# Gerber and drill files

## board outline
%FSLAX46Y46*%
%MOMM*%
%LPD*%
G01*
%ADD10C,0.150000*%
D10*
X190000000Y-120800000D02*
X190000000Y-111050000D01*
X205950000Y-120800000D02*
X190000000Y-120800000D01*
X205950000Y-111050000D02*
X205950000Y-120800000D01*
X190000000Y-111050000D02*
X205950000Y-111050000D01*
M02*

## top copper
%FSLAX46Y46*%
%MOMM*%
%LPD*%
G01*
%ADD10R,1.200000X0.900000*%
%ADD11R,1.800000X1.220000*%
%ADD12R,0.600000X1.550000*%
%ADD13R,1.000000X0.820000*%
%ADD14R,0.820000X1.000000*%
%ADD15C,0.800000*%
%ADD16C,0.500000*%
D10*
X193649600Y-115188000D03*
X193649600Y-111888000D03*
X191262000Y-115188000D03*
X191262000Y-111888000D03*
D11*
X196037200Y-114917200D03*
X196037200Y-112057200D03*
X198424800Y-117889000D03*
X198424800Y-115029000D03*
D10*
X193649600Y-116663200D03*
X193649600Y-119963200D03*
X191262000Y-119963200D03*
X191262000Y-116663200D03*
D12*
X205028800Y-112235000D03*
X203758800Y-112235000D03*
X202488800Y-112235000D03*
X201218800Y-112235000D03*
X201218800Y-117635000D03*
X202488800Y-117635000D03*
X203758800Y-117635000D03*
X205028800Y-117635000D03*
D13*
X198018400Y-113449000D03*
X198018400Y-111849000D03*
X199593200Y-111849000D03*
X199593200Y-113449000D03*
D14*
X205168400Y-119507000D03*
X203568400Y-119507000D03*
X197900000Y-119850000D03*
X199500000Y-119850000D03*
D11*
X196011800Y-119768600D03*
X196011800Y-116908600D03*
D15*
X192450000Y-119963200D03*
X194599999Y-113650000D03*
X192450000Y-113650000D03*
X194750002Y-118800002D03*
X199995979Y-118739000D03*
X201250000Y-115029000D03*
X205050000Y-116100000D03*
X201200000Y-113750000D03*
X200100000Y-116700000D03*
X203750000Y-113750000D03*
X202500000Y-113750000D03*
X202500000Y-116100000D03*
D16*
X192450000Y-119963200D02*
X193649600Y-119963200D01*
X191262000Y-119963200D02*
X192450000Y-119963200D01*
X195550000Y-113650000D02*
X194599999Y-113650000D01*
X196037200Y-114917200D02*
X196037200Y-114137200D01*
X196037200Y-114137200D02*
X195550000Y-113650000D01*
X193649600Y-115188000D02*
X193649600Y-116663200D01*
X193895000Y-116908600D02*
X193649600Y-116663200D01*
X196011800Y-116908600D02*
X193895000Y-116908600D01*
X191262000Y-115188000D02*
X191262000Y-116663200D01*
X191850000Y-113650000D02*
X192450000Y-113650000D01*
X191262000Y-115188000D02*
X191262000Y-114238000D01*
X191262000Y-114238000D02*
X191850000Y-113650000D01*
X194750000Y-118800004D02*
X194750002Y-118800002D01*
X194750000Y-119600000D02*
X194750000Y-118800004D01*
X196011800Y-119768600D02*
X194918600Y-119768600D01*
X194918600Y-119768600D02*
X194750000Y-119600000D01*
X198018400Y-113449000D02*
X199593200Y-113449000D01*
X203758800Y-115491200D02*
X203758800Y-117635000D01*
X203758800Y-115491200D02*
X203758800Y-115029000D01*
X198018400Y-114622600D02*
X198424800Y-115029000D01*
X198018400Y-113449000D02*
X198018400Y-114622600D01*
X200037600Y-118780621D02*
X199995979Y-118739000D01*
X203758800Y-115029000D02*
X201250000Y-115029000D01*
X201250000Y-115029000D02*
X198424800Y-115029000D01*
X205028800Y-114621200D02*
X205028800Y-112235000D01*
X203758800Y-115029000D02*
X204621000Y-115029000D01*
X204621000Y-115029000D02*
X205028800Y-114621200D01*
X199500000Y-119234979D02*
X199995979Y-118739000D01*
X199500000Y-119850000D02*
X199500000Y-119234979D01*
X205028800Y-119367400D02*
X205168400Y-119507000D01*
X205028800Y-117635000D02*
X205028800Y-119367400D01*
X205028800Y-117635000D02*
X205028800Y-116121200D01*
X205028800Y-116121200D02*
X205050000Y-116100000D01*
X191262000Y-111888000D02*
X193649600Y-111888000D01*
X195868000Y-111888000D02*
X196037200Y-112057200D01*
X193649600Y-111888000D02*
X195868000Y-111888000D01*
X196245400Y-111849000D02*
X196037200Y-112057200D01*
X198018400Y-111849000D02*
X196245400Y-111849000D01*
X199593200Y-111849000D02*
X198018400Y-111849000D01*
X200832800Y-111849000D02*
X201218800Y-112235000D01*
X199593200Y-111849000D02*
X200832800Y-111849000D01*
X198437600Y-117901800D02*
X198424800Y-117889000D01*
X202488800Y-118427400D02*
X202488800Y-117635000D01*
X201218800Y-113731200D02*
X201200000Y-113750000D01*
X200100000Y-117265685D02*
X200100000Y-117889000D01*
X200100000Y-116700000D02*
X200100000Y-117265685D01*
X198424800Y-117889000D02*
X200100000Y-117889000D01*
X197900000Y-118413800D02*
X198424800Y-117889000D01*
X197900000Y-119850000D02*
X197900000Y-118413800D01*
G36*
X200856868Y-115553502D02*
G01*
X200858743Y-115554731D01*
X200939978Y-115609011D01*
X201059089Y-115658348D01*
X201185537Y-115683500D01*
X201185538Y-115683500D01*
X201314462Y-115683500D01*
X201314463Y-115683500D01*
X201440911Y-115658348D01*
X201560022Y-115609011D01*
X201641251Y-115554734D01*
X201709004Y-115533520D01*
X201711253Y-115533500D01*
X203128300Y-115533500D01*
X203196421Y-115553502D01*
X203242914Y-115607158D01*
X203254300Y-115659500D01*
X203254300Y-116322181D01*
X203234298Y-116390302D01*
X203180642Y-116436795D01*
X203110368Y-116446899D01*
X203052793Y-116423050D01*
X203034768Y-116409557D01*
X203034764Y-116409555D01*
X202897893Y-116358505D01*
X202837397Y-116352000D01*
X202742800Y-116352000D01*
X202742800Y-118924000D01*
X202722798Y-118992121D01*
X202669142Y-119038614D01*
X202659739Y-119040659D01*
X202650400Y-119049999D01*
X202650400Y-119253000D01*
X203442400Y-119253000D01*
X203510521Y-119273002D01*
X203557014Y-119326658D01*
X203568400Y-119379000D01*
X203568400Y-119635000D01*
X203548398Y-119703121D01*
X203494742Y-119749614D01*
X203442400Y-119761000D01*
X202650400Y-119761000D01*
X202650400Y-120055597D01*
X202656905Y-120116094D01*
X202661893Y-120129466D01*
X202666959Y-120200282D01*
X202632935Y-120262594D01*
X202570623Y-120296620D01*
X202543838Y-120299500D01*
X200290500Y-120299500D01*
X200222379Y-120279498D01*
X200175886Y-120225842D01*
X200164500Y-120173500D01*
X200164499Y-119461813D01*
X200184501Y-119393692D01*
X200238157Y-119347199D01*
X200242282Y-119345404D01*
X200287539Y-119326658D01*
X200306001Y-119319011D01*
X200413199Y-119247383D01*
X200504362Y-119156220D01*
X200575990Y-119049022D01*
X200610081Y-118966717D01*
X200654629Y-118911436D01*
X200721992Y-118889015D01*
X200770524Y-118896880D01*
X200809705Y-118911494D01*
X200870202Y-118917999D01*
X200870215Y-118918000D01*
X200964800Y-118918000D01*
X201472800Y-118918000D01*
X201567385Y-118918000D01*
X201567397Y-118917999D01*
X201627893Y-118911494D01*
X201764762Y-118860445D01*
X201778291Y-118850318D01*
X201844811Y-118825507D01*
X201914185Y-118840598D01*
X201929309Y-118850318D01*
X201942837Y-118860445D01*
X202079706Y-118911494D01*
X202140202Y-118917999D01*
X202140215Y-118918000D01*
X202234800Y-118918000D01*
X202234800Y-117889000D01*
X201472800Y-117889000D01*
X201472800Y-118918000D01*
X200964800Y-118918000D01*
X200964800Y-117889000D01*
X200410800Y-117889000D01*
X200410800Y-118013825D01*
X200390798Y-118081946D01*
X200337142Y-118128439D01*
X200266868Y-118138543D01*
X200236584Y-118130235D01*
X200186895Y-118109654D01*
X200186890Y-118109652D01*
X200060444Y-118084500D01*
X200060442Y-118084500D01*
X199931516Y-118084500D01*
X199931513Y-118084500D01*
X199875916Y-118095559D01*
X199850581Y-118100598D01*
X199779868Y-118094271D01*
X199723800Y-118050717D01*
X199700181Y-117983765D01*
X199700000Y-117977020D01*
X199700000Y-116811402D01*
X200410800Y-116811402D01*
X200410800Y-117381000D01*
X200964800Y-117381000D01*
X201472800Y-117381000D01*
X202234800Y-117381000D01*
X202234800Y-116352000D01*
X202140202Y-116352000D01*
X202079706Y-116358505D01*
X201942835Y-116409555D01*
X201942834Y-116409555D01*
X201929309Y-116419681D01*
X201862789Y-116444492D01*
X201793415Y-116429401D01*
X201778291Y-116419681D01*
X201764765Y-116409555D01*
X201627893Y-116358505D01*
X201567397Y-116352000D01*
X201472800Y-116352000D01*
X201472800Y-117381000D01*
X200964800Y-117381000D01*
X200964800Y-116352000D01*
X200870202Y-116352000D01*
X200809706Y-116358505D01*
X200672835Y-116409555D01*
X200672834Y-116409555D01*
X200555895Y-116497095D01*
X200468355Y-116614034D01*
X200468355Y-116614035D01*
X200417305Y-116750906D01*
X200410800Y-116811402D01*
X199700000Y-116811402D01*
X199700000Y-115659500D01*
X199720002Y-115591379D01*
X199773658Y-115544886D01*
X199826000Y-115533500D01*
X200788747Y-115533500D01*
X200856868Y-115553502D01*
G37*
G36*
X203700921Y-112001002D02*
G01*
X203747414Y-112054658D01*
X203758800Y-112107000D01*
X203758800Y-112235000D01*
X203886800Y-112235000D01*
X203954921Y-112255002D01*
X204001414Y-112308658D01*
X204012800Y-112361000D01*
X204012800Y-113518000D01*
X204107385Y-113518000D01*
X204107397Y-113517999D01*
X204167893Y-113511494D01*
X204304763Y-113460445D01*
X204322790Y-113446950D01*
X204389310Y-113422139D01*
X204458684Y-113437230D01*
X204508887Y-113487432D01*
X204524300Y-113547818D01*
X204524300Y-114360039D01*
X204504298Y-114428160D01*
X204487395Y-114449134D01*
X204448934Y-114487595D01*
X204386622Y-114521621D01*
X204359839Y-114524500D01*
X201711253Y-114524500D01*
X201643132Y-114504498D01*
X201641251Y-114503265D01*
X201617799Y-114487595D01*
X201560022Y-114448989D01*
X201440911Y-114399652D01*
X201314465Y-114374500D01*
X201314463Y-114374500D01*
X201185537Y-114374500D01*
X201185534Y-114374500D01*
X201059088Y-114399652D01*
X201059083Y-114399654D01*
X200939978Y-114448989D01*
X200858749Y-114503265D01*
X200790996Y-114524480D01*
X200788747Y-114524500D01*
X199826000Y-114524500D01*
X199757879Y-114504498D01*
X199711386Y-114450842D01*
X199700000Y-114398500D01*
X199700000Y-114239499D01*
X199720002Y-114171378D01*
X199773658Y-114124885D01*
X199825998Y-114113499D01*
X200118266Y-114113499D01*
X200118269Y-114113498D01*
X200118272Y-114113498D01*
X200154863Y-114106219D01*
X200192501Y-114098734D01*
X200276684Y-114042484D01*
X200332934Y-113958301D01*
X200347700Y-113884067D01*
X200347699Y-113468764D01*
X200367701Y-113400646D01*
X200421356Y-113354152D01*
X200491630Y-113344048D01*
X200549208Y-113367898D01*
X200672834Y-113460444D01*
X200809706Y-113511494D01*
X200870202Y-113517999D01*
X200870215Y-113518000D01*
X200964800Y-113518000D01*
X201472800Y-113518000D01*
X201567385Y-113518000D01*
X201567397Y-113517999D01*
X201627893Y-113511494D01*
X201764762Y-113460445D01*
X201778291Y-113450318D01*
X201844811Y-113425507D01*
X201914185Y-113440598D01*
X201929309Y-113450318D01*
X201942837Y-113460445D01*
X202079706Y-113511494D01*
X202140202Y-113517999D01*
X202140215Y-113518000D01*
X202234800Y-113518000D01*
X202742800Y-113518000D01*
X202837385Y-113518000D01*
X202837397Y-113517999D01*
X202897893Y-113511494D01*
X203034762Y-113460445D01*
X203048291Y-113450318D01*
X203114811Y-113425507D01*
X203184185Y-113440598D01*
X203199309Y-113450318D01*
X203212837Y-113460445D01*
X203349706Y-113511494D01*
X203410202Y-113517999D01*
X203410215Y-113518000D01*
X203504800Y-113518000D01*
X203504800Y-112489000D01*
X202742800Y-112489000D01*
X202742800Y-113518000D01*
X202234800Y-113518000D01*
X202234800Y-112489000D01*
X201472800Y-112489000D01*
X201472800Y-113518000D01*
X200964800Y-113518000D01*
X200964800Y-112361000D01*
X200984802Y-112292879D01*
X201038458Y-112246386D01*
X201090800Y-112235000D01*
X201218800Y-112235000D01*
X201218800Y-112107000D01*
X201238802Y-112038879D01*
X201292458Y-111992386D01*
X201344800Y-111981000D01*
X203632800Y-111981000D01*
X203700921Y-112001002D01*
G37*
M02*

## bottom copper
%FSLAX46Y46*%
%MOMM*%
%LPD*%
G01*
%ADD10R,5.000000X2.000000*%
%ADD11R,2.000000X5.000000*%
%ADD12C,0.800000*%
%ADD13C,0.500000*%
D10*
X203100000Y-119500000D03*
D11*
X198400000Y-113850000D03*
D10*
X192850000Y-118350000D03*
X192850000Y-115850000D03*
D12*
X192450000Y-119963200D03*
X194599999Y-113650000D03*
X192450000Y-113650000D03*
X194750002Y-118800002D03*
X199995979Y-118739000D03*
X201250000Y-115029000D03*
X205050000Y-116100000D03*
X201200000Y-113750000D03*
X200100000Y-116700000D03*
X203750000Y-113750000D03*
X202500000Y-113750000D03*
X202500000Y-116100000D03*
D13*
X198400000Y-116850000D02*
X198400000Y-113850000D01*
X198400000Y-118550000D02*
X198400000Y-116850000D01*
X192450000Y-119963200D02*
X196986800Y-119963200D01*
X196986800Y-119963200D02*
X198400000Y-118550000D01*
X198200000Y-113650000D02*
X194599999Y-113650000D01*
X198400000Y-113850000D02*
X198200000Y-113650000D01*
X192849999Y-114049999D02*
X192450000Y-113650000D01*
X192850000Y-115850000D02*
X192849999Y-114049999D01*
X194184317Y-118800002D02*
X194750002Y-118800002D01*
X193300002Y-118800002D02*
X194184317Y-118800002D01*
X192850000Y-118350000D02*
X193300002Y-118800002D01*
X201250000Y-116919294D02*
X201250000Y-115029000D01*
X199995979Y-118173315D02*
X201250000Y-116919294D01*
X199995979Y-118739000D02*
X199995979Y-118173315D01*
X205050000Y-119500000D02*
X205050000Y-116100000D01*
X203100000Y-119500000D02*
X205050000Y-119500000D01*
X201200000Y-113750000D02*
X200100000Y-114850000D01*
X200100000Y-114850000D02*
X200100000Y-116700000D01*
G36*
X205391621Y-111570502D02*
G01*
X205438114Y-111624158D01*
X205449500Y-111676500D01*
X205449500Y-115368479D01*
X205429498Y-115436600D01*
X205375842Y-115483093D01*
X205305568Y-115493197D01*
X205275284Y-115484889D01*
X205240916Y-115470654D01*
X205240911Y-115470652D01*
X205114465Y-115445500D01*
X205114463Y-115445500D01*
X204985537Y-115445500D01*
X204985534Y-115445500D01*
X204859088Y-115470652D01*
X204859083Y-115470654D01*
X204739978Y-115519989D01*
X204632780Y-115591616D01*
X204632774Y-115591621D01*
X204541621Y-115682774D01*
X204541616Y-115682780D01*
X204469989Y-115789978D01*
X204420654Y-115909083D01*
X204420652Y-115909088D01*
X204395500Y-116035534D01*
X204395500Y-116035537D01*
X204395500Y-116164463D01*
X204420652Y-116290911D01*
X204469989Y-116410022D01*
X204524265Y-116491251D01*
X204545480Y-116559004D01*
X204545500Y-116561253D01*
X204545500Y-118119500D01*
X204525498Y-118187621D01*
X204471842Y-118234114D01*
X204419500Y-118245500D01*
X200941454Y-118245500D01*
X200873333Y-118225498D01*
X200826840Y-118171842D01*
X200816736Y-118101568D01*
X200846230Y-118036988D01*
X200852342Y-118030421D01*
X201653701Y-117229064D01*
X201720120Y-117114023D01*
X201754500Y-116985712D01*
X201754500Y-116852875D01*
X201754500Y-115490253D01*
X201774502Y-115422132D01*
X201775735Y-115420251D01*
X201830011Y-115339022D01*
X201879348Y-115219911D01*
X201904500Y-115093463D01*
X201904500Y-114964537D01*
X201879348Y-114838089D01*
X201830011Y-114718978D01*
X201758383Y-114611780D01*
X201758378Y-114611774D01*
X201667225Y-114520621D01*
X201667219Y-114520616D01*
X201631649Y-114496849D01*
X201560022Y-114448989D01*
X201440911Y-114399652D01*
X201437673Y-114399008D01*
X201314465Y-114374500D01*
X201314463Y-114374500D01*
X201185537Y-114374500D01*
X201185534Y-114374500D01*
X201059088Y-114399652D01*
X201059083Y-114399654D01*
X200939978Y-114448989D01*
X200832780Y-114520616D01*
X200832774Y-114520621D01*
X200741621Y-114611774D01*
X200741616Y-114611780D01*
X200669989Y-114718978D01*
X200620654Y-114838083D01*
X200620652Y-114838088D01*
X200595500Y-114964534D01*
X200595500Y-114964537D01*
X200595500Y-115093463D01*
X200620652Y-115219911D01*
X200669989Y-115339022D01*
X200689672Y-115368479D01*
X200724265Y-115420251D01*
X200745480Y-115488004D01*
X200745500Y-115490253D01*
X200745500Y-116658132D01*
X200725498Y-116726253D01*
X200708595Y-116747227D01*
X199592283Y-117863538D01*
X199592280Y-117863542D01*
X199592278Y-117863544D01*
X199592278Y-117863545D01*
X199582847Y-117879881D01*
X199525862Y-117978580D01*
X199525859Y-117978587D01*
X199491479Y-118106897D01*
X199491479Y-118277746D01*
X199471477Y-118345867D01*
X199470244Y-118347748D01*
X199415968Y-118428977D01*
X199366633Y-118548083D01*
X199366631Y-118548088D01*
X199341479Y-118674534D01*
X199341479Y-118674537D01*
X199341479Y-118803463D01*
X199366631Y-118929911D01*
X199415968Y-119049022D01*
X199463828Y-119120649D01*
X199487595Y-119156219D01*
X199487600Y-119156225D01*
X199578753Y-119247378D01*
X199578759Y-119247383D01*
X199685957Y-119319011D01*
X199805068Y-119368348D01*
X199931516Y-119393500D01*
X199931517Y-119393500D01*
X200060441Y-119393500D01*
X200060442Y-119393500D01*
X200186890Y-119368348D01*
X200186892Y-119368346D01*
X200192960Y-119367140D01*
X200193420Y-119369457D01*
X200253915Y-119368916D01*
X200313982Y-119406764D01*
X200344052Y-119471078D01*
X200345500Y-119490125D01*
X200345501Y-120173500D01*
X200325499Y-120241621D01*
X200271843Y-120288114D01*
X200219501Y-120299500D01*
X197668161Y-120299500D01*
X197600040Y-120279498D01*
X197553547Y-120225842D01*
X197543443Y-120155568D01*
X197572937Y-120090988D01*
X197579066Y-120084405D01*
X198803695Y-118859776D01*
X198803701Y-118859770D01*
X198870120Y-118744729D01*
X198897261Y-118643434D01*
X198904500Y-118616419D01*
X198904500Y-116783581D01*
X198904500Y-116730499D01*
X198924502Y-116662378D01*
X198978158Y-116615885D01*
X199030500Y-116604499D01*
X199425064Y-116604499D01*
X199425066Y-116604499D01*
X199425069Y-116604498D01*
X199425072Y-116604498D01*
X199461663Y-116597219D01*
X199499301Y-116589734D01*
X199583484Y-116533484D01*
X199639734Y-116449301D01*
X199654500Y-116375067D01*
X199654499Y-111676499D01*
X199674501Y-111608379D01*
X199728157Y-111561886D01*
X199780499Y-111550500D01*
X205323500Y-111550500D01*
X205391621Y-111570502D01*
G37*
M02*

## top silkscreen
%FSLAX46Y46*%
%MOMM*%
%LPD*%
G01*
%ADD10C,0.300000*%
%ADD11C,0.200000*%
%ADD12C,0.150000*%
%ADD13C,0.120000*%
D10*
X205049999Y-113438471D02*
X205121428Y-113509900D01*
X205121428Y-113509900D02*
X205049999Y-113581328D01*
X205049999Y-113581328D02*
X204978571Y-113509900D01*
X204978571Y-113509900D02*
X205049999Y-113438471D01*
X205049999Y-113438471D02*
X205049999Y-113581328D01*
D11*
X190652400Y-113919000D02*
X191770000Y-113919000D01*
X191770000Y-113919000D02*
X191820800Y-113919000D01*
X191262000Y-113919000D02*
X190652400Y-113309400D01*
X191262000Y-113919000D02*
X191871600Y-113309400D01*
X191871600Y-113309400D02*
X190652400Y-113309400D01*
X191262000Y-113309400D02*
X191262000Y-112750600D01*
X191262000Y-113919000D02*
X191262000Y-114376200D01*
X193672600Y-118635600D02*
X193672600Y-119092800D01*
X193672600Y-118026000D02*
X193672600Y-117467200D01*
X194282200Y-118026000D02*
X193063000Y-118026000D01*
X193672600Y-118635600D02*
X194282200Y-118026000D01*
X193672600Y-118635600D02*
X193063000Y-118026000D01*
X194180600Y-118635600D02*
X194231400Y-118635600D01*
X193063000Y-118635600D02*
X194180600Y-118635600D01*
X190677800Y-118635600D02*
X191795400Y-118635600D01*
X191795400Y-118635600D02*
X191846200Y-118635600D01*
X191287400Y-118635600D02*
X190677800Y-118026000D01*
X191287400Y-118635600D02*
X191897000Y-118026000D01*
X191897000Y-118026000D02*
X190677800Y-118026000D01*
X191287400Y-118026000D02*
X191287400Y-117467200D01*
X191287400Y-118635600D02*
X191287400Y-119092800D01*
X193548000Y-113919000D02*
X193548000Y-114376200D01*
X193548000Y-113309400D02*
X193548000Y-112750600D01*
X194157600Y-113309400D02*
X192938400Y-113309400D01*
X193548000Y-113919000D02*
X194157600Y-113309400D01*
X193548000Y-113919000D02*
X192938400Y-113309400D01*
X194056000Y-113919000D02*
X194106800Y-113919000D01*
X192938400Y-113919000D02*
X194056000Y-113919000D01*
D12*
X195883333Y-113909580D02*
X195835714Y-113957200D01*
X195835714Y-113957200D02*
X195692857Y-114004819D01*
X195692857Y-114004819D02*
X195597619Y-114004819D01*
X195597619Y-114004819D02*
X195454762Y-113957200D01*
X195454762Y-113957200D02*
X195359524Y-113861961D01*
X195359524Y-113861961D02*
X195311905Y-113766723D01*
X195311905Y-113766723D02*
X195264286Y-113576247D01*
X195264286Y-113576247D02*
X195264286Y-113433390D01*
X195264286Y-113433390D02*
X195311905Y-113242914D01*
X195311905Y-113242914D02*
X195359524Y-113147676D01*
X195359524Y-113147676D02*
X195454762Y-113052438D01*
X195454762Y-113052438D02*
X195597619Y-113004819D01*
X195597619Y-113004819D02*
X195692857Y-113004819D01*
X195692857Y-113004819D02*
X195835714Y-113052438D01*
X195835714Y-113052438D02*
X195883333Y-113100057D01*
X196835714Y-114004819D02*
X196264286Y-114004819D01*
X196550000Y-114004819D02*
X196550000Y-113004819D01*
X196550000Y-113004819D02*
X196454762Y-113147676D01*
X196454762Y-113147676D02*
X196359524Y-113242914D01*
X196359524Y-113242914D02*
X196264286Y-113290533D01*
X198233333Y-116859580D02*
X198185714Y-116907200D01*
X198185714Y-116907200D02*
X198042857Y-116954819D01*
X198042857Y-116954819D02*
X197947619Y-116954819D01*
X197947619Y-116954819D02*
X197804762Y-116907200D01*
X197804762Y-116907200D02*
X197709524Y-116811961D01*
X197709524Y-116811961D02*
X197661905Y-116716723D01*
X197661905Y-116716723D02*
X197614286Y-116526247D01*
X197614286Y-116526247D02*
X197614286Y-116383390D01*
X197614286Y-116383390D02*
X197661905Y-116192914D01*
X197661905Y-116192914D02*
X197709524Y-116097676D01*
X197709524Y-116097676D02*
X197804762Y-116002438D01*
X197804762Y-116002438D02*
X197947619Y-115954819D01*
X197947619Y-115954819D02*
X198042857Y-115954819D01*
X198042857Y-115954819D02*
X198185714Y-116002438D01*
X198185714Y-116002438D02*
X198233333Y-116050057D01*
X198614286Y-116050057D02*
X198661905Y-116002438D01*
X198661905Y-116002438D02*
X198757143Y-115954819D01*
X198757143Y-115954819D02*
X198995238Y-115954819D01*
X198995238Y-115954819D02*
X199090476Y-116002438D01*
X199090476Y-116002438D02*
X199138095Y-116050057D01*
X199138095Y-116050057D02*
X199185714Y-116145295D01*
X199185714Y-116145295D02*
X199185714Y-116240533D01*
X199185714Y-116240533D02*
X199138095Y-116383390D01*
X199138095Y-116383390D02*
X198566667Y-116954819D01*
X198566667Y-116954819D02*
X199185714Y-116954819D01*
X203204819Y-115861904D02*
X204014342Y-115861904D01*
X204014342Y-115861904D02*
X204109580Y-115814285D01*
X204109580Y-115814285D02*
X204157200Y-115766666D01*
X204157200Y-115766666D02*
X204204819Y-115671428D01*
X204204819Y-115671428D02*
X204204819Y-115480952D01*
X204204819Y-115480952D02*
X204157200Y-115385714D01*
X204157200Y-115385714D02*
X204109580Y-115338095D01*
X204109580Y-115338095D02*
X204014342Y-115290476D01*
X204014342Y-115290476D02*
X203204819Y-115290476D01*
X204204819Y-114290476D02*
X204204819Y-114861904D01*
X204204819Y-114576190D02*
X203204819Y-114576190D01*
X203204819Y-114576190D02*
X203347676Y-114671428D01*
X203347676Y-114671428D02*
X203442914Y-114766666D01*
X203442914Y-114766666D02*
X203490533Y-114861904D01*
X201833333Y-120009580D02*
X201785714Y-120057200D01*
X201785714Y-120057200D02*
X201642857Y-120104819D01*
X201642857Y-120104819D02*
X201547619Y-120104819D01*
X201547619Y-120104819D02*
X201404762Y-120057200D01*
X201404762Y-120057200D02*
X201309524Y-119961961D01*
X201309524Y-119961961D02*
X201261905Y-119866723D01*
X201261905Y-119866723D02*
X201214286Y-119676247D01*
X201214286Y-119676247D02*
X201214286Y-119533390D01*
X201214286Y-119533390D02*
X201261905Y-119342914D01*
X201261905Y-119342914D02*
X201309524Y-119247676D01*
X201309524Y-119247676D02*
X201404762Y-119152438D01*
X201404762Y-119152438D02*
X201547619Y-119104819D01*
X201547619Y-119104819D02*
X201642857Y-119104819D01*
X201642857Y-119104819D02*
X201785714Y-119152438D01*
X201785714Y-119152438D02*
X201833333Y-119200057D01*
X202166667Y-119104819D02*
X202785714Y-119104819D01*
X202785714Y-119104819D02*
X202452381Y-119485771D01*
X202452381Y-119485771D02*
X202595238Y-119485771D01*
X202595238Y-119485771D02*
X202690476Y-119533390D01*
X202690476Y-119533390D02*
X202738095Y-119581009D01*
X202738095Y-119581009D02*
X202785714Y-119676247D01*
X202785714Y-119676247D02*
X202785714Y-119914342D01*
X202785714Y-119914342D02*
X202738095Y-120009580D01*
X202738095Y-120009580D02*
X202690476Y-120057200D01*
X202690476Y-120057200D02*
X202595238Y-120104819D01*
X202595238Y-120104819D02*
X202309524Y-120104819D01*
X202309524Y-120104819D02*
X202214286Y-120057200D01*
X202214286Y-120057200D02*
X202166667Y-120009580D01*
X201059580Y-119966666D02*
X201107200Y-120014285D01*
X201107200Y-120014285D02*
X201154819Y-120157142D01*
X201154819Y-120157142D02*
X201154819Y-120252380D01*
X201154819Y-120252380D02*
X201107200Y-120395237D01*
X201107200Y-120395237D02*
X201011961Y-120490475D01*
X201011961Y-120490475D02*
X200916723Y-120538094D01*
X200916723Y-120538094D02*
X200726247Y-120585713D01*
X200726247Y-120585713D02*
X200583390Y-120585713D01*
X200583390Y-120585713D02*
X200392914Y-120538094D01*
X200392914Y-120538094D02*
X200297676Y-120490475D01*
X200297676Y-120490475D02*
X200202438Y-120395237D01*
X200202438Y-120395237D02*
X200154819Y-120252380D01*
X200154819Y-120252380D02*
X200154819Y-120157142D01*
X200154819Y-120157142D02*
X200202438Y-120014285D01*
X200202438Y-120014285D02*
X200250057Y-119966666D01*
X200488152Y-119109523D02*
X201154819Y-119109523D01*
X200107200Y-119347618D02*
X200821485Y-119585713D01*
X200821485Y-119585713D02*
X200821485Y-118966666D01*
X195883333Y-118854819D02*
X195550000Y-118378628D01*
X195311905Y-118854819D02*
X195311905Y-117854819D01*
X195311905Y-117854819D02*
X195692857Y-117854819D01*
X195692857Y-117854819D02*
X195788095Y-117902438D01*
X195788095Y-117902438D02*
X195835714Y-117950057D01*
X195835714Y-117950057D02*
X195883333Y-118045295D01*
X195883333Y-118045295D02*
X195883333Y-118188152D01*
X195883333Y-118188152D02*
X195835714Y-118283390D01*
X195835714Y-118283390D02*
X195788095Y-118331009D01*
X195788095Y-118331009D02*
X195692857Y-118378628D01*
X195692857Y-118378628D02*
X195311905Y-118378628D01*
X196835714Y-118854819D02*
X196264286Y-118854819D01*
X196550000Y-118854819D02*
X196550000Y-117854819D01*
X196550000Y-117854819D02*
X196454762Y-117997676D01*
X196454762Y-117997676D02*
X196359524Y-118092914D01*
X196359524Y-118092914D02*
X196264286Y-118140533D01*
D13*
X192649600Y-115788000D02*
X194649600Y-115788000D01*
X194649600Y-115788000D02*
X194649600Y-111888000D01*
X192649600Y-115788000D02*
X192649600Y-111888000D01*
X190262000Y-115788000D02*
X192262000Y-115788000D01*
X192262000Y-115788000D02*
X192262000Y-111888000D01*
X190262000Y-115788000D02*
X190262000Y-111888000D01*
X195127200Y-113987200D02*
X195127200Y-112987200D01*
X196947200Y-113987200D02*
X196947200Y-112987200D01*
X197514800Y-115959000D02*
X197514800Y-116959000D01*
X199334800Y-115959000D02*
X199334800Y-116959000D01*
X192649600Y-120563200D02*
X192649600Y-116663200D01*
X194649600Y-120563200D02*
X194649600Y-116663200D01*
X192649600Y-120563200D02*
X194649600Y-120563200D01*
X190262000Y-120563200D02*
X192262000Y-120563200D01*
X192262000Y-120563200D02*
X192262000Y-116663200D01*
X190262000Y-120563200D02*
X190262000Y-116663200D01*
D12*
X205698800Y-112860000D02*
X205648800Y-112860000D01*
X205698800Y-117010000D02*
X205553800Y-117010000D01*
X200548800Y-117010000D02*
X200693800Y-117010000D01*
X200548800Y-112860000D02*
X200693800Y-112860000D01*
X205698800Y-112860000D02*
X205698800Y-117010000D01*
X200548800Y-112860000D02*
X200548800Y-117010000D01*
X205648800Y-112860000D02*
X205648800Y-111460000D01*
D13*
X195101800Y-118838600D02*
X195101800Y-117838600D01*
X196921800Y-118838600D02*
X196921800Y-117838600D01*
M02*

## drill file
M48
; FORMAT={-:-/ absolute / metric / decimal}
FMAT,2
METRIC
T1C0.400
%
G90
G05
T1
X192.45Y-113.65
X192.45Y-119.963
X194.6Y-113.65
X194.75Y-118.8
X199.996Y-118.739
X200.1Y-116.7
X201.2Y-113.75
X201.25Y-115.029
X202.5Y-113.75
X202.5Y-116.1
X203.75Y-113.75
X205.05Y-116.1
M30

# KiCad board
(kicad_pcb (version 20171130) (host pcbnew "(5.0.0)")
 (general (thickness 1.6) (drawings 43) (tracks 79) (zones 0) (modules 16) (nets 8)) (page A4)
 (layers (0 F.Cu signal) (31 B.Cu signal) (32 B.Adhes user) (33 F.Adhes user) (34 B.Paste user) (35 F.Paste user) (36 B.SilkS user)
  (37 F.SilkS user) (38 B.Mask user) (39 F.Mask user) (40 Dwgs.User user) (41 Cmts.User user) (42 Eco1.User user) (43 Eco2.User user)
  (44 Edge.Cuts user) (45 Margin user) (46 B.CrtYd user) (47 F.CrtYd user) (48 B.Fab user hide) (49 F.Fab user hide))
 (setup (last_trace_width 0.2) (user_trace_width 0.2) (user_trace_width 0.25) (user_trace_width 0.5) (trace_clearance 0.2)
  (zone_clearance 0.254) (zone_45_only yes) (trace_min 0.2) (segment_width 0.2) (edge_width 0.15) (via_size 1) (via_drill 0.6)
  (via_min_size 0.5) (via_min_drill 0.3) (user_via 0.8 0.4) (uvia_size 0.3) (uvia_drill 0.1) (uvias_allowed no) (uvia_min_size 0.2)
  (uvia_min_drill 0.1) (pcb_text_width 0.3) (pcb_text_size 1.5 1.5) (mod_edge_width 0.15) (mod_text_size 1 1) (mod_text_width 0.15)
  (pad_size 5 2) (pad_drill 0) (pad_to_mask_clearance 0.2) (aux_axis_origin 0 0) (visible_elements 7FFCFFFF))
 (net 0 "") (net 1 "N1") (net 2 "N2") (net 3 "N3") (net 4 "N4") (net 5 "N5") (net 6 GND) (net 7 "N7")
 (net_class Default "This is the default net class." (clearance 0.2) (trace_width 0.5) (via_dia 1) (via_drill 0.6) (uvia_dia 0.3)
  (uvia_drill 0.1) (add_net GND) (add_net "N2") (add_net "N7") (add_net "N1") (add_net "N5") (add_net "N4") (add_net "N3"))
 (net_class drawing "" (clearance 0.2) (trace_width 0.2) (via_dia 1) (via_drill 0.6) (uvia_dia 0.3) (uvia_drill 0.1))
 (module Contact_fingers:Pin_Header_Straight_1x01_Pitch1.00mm (layer F.Cu) (at 203.1 119.5)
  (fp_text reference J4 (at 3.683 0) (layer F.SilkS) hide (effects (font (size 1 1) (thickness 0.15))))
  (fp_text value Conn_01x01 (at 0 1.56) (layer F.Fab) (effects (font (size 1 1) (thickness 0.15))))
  (pad 1 smd rect (at 0 0) (size 5 2) (layers B.Cu) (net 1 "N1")))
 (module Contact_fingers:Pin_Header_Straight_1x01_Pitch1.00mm (layer F.Cu) (at 198.4 113.85 270)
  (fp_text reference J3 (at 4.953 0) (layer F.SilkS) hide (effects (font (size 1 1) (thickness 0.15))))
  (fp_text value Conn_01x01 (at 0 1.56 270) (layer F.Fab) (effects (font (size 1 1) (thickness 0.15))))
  (pad 1 smd rect (at 0 0 270) (size 5 2) (layers B.Cu) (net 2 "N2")))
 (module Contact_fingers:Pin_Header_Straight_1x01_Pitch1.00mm (layer F.Cu) (at 192.85 118.35)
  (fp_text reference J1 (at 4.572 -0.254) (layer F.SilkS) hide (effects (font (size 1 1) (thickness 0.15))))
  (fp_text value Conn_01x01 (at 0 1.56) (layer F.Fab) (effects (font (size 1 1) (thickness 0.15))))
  (pad 1 smd rect (at 0 0) (size 5 2) (layers B.Cu) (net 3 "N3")))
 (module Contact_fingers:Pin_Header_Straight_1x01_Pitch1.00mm (layer F.Cu) (at 192.85 115.85)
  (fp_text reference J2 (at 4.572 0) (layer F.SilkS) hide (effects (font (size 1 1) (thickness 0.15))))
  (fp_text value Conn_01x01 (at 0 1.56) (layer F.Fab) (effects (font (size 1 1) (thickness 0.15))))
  (pad 1 smd rect (at 0 0) (size 5 2) (layers B.Cu) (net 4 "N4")))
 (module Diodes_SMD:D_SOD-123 (layer F.Cu) (at 193.6496 113.538 90)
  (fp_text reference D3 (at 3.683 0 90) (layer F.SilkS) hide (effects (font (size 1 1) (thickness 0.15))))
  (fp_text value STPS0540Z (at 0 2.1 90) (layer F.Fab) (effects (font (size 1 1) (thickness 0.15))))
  (fp_line (start -2.25 -1) (end -2.25 1) (layer F.SilkS) (width 0.12))
  (fp_line (start -2.25 1) (end 1.65 1) (layer F.SilkS) (width 0.12))
  (fp_line (start -2.25 -1) (end 1.65 -1) (layer F.SilkS) (width 0.12))
  (pad 1 smd rect (at -1.65 0 90) (size 0.9 1.2) (layers F.Cu F.Paste F.Mask) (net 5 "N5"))
  (pad 2 smd rect (at 1.65 0 90) (size 0.9 1.2) (layers F.Cu F.Paste F.Mask) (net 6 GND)))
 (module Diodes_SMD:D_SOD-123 (layer F.Cu) (at 191.262 113.538 90)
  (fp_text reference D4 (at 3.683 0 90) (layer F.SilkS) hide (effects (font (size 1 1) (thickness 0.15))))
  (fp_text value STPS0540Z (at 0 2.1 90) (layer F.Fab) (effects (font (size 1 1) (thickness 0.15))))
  (fp_line (start -2.25 -1) (end -2.25 1) (layer F.SilkS) (width 0.12))
  (fp_line (start -2.25 1) (end 1.65 1) (layer F.SilkS) (width 0.12))
  (fp_line (start -2.25 -1) (end 1.65 -1) (layer F.SilkS) (width 0.12))
  (pad 1 smd rect (at -1.65 0 90) (size 0.9 1.2) (layers F.Cu F.Paste F.Mask) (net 4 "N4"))
  (pad 2 smd rect (at 1.65 0 90) (size 0.9 1.2) (layers F.Cu F.Paste F.Mask) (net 6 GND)))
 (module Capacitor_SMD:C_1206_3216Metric (layer F.Cu) (at 196.0372 113.4872 90)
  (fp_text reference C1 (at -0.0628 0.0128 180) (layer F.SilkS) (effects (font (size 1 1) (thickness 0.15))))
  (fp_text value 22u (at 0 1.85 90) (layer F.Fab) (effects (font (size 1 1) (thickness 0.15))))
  (fp_line (start -0.5 -0.91) (end 0.5 -0.91) (layer F.SilkS) (width 0.12))
  (fp_line (start -0.5 0.91) (end 0.5 0.91) (layer F.SilkS) (width 0.12))
  (pad 1 smd rect (at -1.43 0 90) (size 1.22 1.8) (layers F.Cu F.Paste F.Mask) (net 2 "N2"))
  (pad 2 smd rect (at 1.43 0 90) (size 1.22 1.8) (layers F.Cu F.Paste F.Mask) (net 6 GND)))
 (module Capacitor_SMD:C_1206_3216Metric (layer F.Cu) (at 198.4248 116.459 270)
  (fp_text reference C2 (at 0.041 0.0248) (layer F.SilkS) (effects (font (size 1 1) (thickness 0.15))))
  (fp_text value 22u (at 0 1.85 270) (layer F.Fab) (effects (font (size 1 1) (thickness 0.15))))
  (fp_line (start -0.5 0.91) (end 0.5 0.91) (layer F.SilkS) (width 0.12))
  (fp_line (start -0.5 -0.91) (end 0.5 -0.91) (layer F.SilkS) (width 0.12))
  (pad 2 smd rect (at 1.43 0 270) (size 1.22 1.8) (layers F.Cu F.Paste F.Mask) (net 6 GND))
  (pad 1 smd rect (at -1.43 0 270) (size 1.22 1.8) (layers F.Cu F.Paste F.Mask) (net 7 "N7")))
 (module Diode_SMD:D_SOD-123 (layer F.Cu) (at 193.6496 118.3132 90)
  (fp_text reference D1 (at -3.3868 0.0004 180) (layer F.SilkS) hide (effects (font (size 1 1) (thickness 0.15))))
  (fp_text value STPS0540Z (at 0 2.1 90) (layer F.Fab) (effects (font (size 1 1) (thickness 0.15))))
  (fp_line (start -2.25 -1) (end 1.65 -1) (layer F.SilkS) (width 0.12))
  (fp_line (start -2.25 1) (end 1.65 1) (layer F.SilkS) (width 0.12))
  (fp_line (start -2.25 -1) (end -2.25 1) (layer F.SilkS) (width 0.12))
  (pad 2 smd rect (at 1.65 0 90) (size 0.9 1.2) (layers F.Cu F.Paste F.Mask) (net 5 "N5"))
  (pad 1 smd rect (at -1.65 0 90) (size 0.9 1.2) (layers F.Cu F.Paste F.Mask) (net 2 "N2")))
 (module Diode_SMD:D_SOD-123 (layer F.Cu) (at 191.262 118.3132 90)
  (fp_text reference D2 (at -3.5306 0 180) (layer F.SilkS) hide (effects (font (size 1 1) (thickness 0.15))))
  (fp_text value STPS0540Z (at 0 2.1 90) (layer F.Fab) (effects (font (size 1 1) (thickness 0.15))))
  (fp_line (start -2.25 -1) (end -2.25 1) (layer F.SilkS) (width 0.12))
  (fp_line (start -2.25 1) (end 1.65 1) (layer F.SilkS) (width 0.12))
  (fp_line (start -2.25 -1) (end 1.65 -1) (layer F.SilkS) (width 0.12))
  (pad 1 smd rect (at -1.65 0 90) (size 0.9 1.2) (layers F.Cu F.Paste F.Mask) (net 2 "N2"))
  (pad 2 smd rect (at 1.65 0 90) (size 0.9 1.2) (layers F.Cu F.Paste F.Mask) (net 4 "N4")))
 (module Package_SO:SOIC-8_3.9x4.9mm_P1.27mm (layer F.Cu) (at 203.1238 114.935 270)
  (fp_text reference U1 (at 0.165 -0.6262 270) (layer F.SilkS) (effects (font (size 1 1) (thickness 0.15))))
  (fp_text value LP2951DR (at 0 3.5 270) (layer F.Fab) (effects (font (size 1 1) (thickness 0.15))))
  (fp_line (start -2.075 -2.575) (end -2.075 -2.525) (layer F.SilkS) (width 0.15))
  (fp_line (start 2.075 -2.575) (end 2.075 -2.43) (layer F.SilkS) (width 0.15))
  (fp_line (start 2.075 2.575) (end 2.075 2.43) (layer F.SilkS) (width 0.15))
  (fp_line (start -2.075 2.575) (end -2.075 2.43) (layer F.SilkS) (width 0.15))
  (fp_line (start -2.075 -2.575) (end 2.075 -2.575) (layer F.SilkS) (width 0.15))
  (fp_line (start -2.075 2.575) (end 2.075 2.575) (layer F.SilkS) (width 0.15))
  (fp_line (start -2.075 -2.525) (end -3.475 -2.525) (layer F.SilkS) (width 0.15))
  (pad 1 smd rect (at -2.7 -1.905 270) (size 1.55 0.6) (layers F.Cu F.Paste F.Mask) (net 7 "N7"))
  (pad 2 smd rect (at -2.7 -0.635 270) (size 1.55 0.6) (layers F.Cu F.Paste F.Mask) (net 6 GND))
  (pad 3 smd rect (at -2.7 0.635 270) (size 1.55 0.6) (layers F.Cu F.Paste F.Mask) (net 6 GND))
  (pad 4 smd rect (at -2.7 1.905 270) (size 1.55 0.6) (layers F.Cu F.Paste F.Mask) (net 6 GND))
  (pad 5 smd rect (at 2.7 1.905 270) (size 1.55 0.6) (layers F.Cu F.Paste F.Mask) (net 6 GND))
  (pad 6 smd rect (at 2.7 0.635 270) (size 1.55 0.6) (layers F.Cu F.Paste F.Mask) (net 6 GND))
  (pad 7 smd rect (at 2.7 -0.635 270) (size 1.55 0.6) (layers F.Cu F.Paste F.Mask) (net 7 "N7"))
  (pad 8 smd rect (at 2.7 -1.905 270) (size 1.55 0.6) (layers F.Cu F.Paste F.Mask) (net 1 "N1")))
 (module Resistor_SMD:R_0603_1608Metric (layer F.Cu) (at 198.0184 112.649 270)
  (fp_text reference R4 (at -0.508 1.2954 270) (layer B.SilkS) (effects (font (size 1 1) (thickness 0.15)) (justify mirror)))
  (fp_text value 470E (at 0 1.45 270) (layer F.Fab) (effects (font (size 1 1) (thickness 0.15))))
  (pad 2 smd rect (at 0.8 0 270) (size 0.82 1) (layers F.Cu F.Paste F.Mask) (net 7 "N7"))
  (pad 1 smd rect (at -0.8 0 270) (size 0.82 1) (layers F.Cu F.Paste F.Mask) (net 6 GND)))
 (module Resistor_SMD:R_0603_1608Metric (layer F.Cu) (at 199.5932 112.649 270)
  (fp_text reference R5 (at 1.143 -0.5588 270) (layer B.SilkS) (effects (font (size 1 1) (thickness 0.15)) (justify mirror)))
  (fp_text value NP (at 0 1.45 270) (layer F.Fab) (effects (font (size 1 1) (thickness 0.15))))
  (pad 1 smd rect (at -0.8 0 270) (size 0.82 1) (layers F.Cu F.Paste F.Mask) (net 6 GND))
  (pad 2 smd rect (at 0.8 0 270) (size 0.82 1) (layers F.Cu F.Paste F.Mask) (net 7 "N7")))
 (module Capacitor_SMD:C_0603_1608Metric (layer F.Cu) (at 204.3684 119.507 180)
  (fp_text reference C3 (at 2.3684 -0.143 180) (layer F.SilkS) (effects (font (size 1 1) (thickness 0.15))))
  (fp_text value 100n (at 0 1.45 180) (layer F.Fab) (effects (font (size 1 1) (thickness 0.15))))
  (pad 1 smd rect (at -0.8 0 180) (size 0.82 1) (layers F.Cu F.Paste F.Mask) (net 1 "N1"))
  (pad 2 smd rect (at 0.8 0 180) (size 0.82 1) (layers F.Cu F.Paste F.Mask) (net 6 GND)))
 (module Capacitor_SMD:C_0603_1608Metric (layer F.Cu) (at 198.7 119.85 180)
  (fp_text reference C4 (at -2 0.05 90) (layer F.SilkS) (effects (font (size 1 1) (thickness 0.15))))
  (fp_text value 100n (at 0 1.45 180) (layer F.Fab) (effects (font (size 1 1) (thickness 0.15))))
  (pad 2 smd rect (at 0.8 0 180) (size 0.82 1) (layers F.Cu F.Paste F.Mask) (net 6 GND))
  (pad 1 smd rect (at -0.8 0 180) (size 0.82 1) (layers F.Cu F.Paste F.Mask) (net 7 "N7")))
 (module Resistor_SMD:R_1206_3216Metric (layer F.Cu) (at 196.0118 118.3386 90)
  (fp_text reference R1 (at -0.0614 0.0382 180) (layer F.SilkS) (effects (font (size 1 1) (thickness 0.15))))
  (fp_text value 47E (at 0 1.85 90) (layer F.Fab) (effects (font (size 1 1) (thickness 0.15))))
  (fp_line (start -0.5 -0.91) (end 0.5 -0.91) (layer F.SilkS) (width 0.12))
  (fp_line (start -0.5 0.91) (end 0.5 0.91) (layer F.SilkS) (width 0.12))
  (pad 1 smd rect (at -1.43 0 90) (size 1.22 1.8) (layers F.Cu F.Paste F.Mask) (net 3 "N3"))
  (pad 2 smd rect (at 1.43 0 90) (size 1.22 1.8) (layers F.Cu F.Paste F.Mask) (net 5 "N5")))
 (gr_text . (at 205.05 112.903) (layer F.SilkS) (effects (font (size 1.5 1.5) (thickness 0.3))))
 (gr_line (start 190 120.8) (end 190 111.05) (layer Edge.Cuts) (width 0.15))
 (gr_line (start 205.95 120.8) (end 190 120.8) (layer Edge.Cuts) (width 0.15))
 (gr_line (start 205.95 111.05) (end 205.95 120.8) (layer Edge.Cuts) (width 0.15))
 (gr_line (start 190 111.05) (end 205.95 111.05) (layer Edge.Cuts) (width 0.15))
 (gr_line (start 190.6524 113.919) (end 191.77 113.919) (angle 90) (layer F.SilkS) (width 0.2))
 (gr_line (start 191.77 113.919) (end 191.8208 113.919) (angle 90) (layer F.SilkS) (width 0.2))
 (gr_line (start 191.262 113.919) (end 190.6524 113.3094) (angle 90) (layer F.SilkS) (width 0.2))
 (gr_line (start 191.262 113.919) (end 191.8716 113.3094) (angle 90) (layer F.SilkS) (width 0.2))
 (gr_line (start 191.8716 113.3094) (end 190.6524 113.3094) (angle 90) (layer F.SilkS) (width 0.2))
 (gr_line (start 191.262 113.3094) (end 191.262 112.7506) (angle 90) (layer F.SilkS) (width 0.2))
 (gr_line (start 191.262 113.919) (end 191.262 114.3762) (angle 90) (layer F.SilkS) (width 0.2))
 (gr_line (start 193.6726 118.6356) (end 193.6726 119.0928) (angle 90) (layer F.SilkS) (width 0.2))
 (gr_line (start 193.6726 118.026) (end 193.6726 117.4672) (angle 90) (layer F.SilkS) (width 0.2))
 (gr_line (start 194.2822 118.026) (end 193.063 118.026) (angle 90) (layer F.SilkS) (width 0.2))
 (gr_line (start 193.6726 118.6356) (end 194.2822 118.026) (angle 90) (layer F.SilkS) (width 0.2))
 (gr_line (start 193.6726 118.6356) (end 193.063 118.026) (angle 90) (layer F.SilkS) (width 0.2))
 (gr_line (start 194.1806 118.6356) (end 194.2314 118.6356) (angle 90) (layer F.SilkS) (width 0.2))
 (gr_line (start 193.063 118.6356) (end 194.1806 118.6356) (angle 90) (layer F.SilkS) (width 0.2))
 (gr_line (start 190.6778 118.6356) (end 191.7954 118.6356) (angle 90) (layer F.SilkS) (width 0.2))
 (gr_line (start 191.7954 118.6356) (end 191.8462 118.6356) (angle 90) (layer F.SilkS) (width 0.2))
 (gr_line (start 191.2874 118.6356) (end 190.6778 118.026) (angle 90) (layer F.SilkS) (width 0.2))
 (gr_line (start 191.2874 118.6356) (end 191.897 118.026) (angle 90) (layer F.SilkS) (width 0.2))
 (gr_line (start 191.897 118.026) (end 190.6778 118.026) (angle 90) (layer F.SilkS) (width 0.2))
 (gr_line (start 191.2874 118.026) (end 191.2874 117.4672) (angle 90) (layer F.SilkS) (width 0.2))
 (gr_line (start 191.2874 118.6356) (end 191.2874 119.0928) (angle 90) (layer F.SilkS) (width 0.2))
 (gr_line (start 193.548 113.919) (end 193.548 114.3762) (angle 90) (layer F.SilkS) (width 0.2))
 (gr_line (start 193.548 113.3094) (end 193.548 112.7506) (angle 90) (layer F.SilkS) (width 0.2))
 (gr_line (start 194.1576 113.3094) (end 192.9384 113.3094) (angle 90) (layer F.SilkS) (width 0.2))
 (gr_line (start 193.548 113.919) (end 194.1576 113.3094) (angle 90) (layer F.SilkS) (width 0.2))
 (gr_line (start 193.548 113.919) (end 192.9384 113.3094) (angle 90) (layer F.SilkS) (width 0.2))
 (gr_line (start 194.056 113.919) (end 194.1068 113.919) (angle 90) (layer F.SilkS) (width 0.2))
 (gr_line (start 192.9384 113.919) (end 194.056 113.919) (angle 90) (layer F.SilkS) (width 0.2))
 (via (at 192.45 119.9632) (size 0.8) (drill 0.4) (layers F.Cu B.Cu) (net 2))
 (segment (start 192.45 119.9632) (end 193.6496 119.9632) (width 0.5) (layer F.Cu) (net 2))
 (segment (start 191.262 119.9632) (end 192.45 119.9632) (width 0.5) (layer F.Cu) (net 2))
 (segment (start 198.4 116.85) (end 198.4 113.85) (width 0.5) (layer B.Cu) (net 2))
 (segment (start 198.4 118.55) (end 198.4 116.85) (width 0.5) (layer B.Cu) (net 2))
 (segment (start 192.45 119.9632) (end 196.9868 119.9632) (width 0.5) (layer B.Cu) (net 2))
 (segment (start 196.9868 119.9632) (end 198.4 118.55) (width 0.5) (layer B.Cu) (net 2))
 (via (at 194.599999 113.65) (size 0.8) (drill 0.4) (layers F.Cu B.Cu) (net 2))
 (segment (start 195.55 113.65) (end 194.599999 113.65) (width 0.5) (layer F.Cu) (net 2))
 (segment (start 196.0372 114.9172) (end 196.0372 114.1372) (width 0.5) (layer F.Cu) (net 2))
 (segment (start 196.0372 114.1372) (end 195.55 113.65) (width 0.5) (layer F.Cu) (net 2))
 (segment (start 198.2 113.65) (end 194.599999 113.65) (width 0.5) (layer B.Cu) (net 2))
 (segment (start 198.4 113.85) (end 198.2 113.65) (width 0.5) (layer B.Cu) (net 2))
 (segment (start 193.6496 115.188) (end 193.6496 116.6632) (width 0.5) (layer F.Cu) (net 5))
 (segment (start 193.895 116.9086) (end 193.6496 116.6632) (width 0.5) (layer F.Cu) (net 5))
 (segment (start 196.0118 116.9086) (end 193.895 116.9086) (width 0.5) (layer F.Cu) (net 5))
 (segment (start 191.262 115.188) (end 191.262 116.6632) (width 0.5) (layer F.Cu) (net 4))
 (via (at 192.45 113.65) (size 0.8) (drill 0.4) (layers F.Cu B.Cu) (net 4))
 (segment (start 192.849999 114.049999) (end 192.45 113.65) (width 0.5) (layer B.Cu) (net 4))
 (segment (start 192.85 115.85) (end 192.849999 114.049999) (width 0.5) (layer B.Cu) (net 4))
 (segment (start 191.85 113.65) (end 192.45 113.65) (width 0.5) (layer F.Cu) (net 4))
 (segment (start 191.262 115.188) (end 191.262 114.238) (width 0.5) (layer F.Cu) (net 4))
 (segment (start 191.262 114.238) (end 191.85 113.65) (width 0.5) (layer F.Cu) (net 4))
 (via (at 194.750002 118.800002) (size 0.8) (drill 0.4) (layers F.Cu B.Cu) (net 3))
 (segment (start 194.184317 118.800002) (end 194.750002 118.800002) (width 0.5) (layer B.Cu) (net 3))
 (segment (start 193.300002 118.800002) (end 194.184317 118.800002) (width 0.5) (layer B.Cu) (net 3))
 (segment (start 192.85 118.35) (end 193.300002 118.800002) (width 0.5) (layer B.Cu) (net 3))
 (segment (start 194.75 118.800004) (end 194.750002 118.800002) (width 0.5) (layer F.Cu) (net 3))
 (segment (start 194.75 119.6) (end 194.75 118.800004) (width 0.5) (layer F.Cu) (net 3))
 (segment (start 196.0118 119.7686) (end 194.9186 119.7686) (width 0.5) (layer F.Cu) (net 3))
 (segment (start 194.9186 119.7686) (end 194.75 119.6) (width 0.5) (layer F.Cu) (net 3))
 (segment (start 198.0184 113.449) (end 199.5932 113.449) (width 0.5) (layer F.Cu) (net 7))
 (segment (start 203.7588 115.4912) (end 203.7588 117.635) (width 0.5) (layer F.Cu) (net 7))
 (segment (start 203.7588 115.4912) (end 203.7588 115.029) (width 0.5) (layer F.Cu) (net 7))
 (segment (start 198.0184 114.6226) (end 198.4248 115.029) (width 0.5) (layer F.Cu) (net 7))
 (segment (start 198.0184 113.449) (end 198.0184 114.6226) (width 0.5) (layer F.Cu) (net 7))
 (via (at 199.995979 118.739) (size 0.8) (drill 0.4) (layers F.Cu B.Cu) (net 7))
 (segment (start 200.0376 118.780621) (end 199.995979 118.739) (width 0.5) (layer F.Cu) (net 7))
 (via (at 201.25 115.029) (size 0.8) (drill 0.4) (layers F.Cu B.Cu) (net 7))
 (segment (start 201.25 116.919294) (end 201.25 115.029) (width 0.5) (layer B.Cu) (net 7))
 (segment (start 199.995979 118.173315) (end 201.25 116.919294) (width 0.5) (layer B.Cu) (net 7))
 (segment (start 199.995979 118.739) (end 199.995979 118.173315) (width 0.5) (layer B.Cu) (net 7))
 (segment (start 203.7588 115.029) (end 201.25 115.029) (width 0.5) (layer F.Cu) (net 7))
 (segment (start 201.25 115.029) (end 198.4248 115.029) (width 0.5) (layer F.Cu) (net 7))
 (segment (start 205.0288 114.6212) (end 205.0288 112.235) (width 0.5) (layer F.Cu) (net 7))
 (segment (start 203.7588 115.029) (end 204.621 115.029) (width 0.5) (layer F.Cu) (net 7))
 (segment (start 204.621 115.029) (end 205.0288 114.6212) (width 0.5) (layer F.Cu) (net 7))
 (segment (start 199.5 119.234979) (end 199.995979 118.739) (width 0.5) (layer F.Cu) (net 7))
 (segment (start 199.5 119.85) (end 199.5 119.234979) (width 0.5) (layer F.Cu) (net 7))
 (segment (start 205.0288 119.3674) (end 205.1684 119.507) (width 0.5) (layer F.Cu) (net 1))
 (segment (start 205.0288 117.635) (end 205.0288 119.3674) (width 0.5) (layer F.Cu) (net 1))
 (via (at 205.05 116.1) (size 0.8) (drill 0.4) (layers F.Cu B.Cu) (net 1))
 (segment (start 205.0288 117.635) (end 205.0288 116.1212) (width 0.5) (layer F.Cu) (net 1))
 (segment (start 205.0288 116.1212) (end 205.05 116.1) (width 0.5) (layer F.Cu) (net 1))
 (segment (start 205.05 119.5) (end 205.05 116.1) (width 0.5) (layer B.Cu) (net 1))
 (segment (start 203.1 119.5) (end 205.05 119.5) (width 0.5) (layer B.Cu) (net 1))
 (segment (start 191.262 111.888) (end 193.6496 111.888) (width 0.5) (layer F.Cu) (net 6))
 (segment (start 195.868 111.888) (end 196.0372 112.0572) (width 0.5) (layer F.Cu) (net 6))
 (segment (start 193.6496 111.888) (end 195.868 111.888) (width 0.5) (layer F.Cu) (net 6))
 (segment (start 196.2454 111.849) (end 196.0372 112.0572) (width 0.5) (layer F.Cu) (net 6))
 (segment (start 198.0184 111.849) (end 196.2454 111.849) (width 0.5) (layer F.Cu) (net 6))
 (segment (start 199.5932 111.849) (end 198.0184 111.849) (width 0.5) (layer F.Cu) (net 6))
 (segment (start 200.8328 111.849) (end 201.2188 112.235) (width 0.5) (layer F.Cu) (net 6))
 (segment (start 199.5932 111.849) (end 200.8328 111.849) (width 0.5) (layer F.Cu) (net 6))
 (segment (start 198.4376 117.9018) (end 198.4248 117.889) (width 0.5) (layer F.Cu) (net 6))
 (segment (start 202.4888 118.4274) (end 202.4888 117.635) (width 0.5) (layer F.Cu) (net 6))
 (via (at 201.2 113.75) (size 0.8) (drill 0.4) (layers F.Cu B.Cu) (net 6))
 (segment (start 201.2188 113.7312) (end 201.2 113.75) (width 0.5) (layer F.Cu) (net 6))
 (segment (start 201.2 113.75) (end 200.1 114.85) (width 0.5) (layer B.Cu) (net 6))
 (segment (start 200.1 114.85) (end 200.1 116.7) (width 0.5) (layer B.Cu) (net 6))
 (via (at 200.1 116.7) (size 0.8) (drill 0.4) (layers F.Cu B.Cu) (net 6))
 (segment (start 200.1 117.265685) (end 200.1 117.889) (width 0.5) (layer F.Cu) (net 6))
 (segment (start 200.1 116.7) (end 200.1 117.265685) (width 0.5) (layer F.Cu) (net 6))
 (segment (start 198.4248 117.889) (end 200.1 117.889) (width 0.5) (layer F.Cu) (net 6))
 (via (at 203.75 113.75) (size 0.8) (drill 0.4) (layers F.Cu B.Cu) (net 6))
 (via (at 202.5 113.75) (size 0.8) (drill 0.4) (layers F.Cu B.Cu) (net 6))
 (via (at 202.5 116.1) (size 0.8) (drill 0.4) (layers F.Cu B.Cu) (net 6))
 (segment (start 197.9 118.4138) (end 198.4248 117.889) (width 0.5) (layer F.Cu) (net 6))
 (segment (start 197.9 119.85) (end 197.9 118.4138) (width 0.5) (layer F.Cu) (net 6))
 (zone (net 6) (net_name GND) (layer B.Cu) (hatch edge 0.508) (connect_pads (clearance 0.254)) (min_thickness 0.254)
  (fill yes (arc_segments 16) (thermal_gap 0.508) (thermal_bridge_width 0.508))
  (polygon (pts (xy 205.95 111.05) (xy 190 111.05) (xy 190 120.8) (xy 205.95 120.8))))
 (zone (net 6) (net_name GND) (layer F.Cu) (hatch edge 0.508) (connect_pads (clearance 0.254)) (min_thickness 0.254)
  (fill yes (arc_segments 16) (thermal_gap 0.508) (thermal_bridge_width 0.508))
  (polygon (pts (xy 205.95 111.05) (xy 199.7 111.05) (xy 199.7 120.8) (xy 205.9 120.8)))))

